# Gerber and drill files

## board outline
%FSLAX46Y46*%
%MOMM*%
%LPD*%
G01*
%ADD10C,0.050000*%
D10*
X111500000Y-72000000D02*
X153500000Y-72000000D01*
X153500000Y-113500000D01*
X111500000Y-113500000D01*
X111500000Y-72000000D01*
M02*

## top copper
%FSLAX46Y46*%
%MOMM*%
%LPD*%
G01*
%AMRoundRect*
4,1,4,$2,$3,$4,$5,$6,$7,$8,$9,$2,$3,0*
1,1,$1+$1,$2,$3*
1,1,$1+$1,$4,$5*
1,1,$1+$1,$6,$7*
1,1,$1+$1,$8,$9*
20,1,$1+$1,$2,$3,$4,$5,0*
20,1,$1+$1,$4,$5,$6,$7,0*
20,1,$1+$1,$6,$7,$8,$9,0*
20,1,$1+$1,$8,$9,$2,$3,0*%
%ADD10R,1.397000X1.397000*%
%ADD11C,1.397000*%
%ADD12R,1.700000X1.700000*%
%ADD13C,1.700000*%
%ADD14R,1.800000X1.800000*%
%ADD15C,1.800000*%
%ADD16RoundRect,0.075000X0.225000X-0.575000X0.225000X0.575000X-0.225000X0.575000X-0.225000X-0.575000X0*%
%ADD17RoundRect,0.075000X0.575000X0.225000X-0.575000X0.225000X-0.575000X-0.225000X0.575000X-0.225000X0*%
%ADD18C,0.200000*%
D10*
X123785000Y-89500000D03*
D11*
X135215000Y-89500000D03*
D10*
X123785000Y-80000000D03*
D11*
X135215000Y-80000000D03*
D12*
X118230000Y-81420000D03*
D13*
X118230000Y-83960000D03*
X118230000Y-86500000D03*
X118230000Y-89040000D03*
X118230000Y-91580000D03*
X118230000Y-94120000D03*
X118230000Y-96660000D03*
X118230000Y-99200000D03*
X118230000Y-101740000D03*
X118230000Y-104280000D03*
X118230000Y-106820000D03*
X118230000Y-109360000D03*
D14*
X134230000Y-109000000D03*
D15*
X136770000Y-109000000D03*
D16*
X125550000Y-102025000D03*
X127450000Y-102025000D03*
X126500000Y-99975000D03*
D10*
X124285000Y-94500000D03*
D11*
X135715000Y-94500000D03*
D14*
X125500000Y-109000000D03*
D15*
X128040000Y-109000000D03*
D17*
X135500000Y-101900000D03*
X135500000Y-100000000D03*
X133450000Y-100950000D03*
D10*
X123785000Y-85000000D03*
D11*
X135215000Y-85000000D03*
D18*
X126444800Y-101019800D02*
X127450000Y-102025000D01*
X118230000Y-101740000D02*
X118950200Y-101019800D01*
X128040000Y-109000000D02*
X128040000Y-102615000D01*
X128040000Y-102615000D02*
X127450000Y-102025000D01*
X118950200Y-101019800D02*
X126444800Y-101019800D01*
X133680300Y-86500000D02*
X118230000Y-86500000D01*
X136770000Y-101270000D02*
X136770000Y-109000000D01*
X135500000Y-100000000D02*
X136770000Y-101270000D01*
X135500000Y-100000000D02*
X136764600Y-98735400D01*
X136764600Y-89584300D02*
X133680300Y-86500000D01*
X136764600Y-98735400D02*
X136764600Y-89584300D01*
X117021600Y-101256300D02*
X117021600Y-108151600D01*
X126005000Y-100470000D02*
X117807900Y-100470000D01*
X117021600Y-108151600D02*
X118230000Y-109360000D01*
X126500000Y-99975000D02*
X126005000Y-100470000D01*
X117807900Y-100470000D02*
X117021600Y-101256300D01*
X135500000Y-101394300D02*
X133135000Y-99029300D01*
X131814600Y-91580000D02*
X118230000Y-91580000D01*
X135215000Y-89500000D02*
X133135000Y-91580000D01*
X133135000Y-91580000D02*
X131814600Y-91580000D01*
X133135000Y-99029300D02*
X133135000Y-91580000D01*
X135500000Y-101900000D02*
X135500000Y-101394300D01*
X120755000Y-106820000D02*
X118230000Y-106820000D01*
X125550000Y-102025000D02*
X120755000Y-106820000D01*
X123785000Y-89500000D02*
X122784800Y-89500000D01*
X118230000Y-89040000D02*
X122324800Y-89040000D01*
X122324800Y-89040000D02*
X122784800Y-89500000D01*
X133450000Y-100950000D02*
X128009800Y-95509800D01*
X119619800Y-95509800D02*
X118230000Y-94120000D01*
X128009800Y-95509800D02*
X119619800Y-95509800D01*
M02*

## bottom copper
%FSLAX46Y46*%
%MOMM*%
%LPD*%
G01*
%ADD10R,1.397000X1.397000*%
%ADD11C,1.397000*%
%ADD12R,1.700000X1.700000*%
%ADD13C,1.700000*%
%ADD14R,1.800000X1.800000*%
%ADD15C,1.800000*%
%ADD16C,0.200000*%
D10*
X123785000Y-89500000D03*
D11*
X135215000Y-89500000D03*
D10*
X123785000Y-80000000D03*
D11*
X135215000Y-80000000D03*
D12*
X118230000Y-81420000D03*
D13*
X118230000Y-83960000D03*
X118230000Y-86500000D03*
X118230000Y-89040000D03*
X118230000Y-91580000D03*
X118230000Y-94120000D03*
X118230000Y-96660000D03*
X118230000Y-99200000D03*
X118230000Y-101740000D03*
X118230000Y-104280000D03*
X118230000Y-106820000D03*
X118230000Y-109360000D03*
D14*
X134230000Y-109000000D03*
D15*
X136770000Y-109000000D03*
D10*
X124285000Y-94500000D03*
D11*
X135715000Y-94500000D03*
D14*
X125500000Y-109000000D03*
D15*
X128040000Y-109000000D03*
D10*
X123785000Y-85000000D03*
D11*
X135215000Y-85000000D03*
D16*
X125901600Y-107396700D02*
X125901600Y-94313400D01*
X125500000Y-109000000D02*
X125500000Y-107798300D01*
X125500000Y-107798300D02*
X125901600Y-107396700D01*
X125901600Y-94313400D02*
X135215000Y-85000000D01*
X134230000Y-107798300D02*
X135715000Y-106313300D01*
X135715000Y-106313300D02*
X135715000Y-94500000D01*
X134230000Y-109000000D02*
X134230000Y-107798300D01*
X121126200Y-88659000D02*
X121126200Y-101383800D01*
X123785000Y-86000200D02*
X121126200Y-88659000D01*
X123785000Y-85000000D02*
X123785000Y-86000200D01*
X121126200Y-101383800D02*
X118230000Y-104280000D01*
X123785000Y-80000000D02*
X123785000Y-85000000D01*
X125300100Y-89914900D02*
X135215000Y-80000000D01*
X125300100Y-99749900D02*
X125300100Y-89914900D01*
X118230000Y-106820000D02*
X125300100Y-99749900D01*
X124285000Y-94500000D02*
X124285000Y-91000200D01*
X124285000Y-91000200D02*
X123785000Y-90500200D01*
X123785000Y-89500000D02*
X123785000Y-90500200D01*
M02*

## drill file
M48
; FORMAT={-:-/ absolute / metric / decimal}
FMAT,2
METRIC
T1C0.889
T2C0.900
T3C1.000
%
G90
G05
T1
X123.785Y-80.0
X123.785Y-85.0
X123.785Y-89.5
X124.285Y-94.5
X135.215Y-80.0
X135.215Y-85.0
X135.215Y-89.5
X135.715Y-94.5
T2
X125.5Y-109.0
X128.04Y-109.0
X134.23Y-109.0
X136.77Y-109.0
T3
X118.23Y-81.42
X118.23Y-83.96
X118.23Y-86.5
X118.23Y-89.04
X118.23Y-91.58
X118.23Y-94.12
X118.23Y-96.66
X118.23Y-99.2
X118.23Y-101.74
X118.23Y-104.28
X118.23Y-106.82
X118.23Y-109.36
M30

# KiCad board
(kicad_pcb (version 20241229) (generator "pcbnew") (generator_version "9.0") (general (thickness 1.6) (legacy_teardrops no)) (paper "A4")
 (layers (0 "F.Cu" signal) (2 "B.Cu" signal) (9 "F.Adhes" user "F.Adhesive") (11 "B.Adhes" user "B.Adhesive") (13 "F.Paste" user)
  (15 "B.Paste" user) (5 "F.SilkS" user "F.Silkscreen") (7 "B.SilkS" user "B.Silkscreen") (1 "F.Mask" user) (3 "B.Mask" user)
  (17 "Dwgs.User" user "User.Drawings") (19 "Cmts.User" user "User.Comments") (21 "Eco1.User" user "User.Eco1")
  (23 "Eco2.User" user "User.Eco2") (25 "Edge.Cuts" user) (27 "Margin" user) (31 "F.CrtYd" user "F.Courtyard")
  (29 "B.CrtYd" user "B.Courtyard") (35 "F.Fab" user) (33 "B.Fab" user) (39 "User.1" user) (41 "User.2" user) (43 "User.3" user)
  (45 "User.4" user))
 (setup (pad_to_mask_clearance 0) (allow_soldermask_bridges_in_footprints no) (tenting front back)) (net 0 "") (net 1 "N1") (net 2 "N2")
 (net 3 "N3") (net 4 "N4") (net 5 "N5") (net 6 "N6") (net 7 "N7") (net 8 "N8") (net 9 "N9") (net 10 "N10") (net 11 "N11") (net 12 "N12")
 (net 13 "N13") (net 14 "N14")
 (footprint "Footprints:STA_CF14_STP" (layer "F.Cu") (at 123.785 89.5)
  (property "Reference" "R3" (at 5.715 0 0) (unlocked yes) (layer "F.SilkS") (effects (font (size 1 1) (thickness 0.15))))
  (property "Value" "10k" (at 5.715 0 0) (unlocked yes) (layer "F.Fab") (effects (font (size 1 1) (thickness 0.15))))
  (pad "1" thru_hole rect (at 0 0) (size 1.397 1.397) (drill 0.889) (layers "*.Cu" "*.Mask") (remove_unused_layers no) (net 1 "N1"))
  (pad "2" thru_hole circle (at 11.43 0) (size 1.397 1.397) (drill 0.889) (layers "*.Cu" "*.Mask") (remove_unused_layers no) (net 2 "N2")))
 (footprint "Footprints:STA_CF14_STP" (layer "F.Cu") (at 123.785 80)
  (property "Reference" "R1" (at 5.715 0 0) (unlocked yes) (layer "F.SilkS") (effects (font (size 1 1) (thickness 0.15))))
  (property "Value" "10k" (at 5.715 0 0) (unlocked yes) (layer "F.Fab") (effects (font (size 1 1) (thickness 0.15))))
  (pad "1" thru_hole rect (at 0 0) (size 1.397 1.397) (drill 0.889) (layers "*.Cu" "*.Mask") (remove_unused_layers no) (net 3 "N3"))
  (pad "2" thru_hole circle (at 11.43 0) (size 1.397 1.397) (drill 0.889) (layers "*.Cu" "*.Mask") (remove_unused_layers no) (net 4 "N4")))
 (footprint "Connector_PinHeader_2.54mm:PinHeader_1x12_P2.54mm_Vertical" (layer "F.Cu") (at 118.23 81.42)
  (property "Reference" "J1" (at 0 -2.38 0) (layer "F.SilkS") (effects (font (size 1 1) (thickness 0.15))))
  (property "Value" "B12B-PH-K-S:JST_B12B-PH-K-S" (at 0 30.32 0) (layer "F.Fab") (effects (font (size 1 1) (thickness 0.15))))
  (pad "1" thru_hole rect (at 0 0) (size 1.7 1.7) (drill 1) (layers "*.Cu" "*.Mask") (remove_unused_layers no) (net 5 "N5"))
  (pad "2" thru_hole circle (at 0 2.54) (size 1.7 1.7) (drill 1) (layers "*.Cu" "*.Mask") (remove_unused_layers no) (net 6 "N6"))
  (pad "3" thru_hole circle (at 0 5.08) (size 1.7 1.7) (drill 1) (layers "*.Cu" "*.Mask") (remove_unused_layers no) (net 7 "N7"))
  (pad "4" thru_hole circle (at 0 7.62) (size 1.7 1.7) (drill 1) (layers "*.Cu" "*.Mask") (remove_unused_layers no) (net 1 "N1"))
  (pad "5" thru_hole circle (at 0 10.16) (size 1.7 1.7) (drill 1) (layers "*.Cu" "*.Mask") (remove_unused_layers no) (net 2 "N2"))
  (pad "6" thru_hole circle (at 0 12.7) (size 1.7 1.7) (drill 1) (layers "*.Cu" "*.Mask") (remove_unused_layers no) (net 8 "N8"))
  (pad "7" thru_hole circle (at 0 15.24) (size 1.7 1.7) (drill 1) (layers "*.Cu" "*.Mask") (remove_unused_layers no) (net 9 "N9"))
  (pad "8" thru_hole circle (at 0 17.78) (size 1.7 1.7) (drill 1) (layers "*.Cu" "*.Mask") (remove_unused_layers no) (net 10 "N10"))
  (pad "9" thru_hole circle (at 0 20.32) (size 1.7 1.7) (drill 1) (layers "*.Cu" "*.Mask") (remove_unused_layers no) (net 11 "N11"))
  (pad "10" thru_hole circle (at 0 22.86) (size 1.7 1.7) (drill 1) (layers "*.Cu" "*.Mask") (remove_unused_layers no) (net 3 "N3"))
  (pad "11" thru_hole circle (at 0 25.4) (size 1.7 1.7) (drill 1) (layers "*.Cu" "*.Mask") (remove_unused_layers no) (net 4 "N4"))
  (pad "12" thru_hole circle (at 0 27.94) (size 1.7 1.7) (drill 1) (layers "*.Cu" "*.Mask") (remove_unused_layers no) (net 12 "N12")))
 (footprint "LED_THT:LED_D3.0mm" (layer "F.Cu") (at 134.23 109)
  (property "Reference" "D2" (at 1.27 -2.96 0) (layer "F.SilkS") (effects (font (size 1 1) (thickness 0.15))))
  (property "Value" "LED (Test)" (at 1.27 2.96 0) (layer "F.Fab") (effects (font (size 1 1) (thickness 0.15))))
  (pad "1" thru_hole rect (at 0 0) (size 1.8 1.8) (drill 0.9) (layers "*.Cu" "*.Mask") (remove_unused_layers no) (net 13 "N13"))
  (pad "2" thru_hole circle (at 2.54 0) (size 1.8 1.8) (drill 0.9) (layers "*.Cu" "*.Mask") (remove_unused_layers no) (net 7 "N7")))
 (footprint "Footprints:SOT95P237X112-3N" (layer "F.Cu") (at 126.5 101 90)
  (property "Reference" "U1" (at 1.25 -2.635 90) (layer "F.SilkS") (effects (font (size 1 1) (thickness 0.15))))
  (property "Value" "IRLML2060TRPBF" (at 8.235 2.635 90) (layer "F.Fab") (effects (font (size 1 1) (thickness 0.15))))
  (pad "1" smd roundrect (at -1.025 -0.95 90) (size 1.3 0.6) (layers "F.Cu" "F.Mask" "F.Paste") (roundrect_rratio 0.125) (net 4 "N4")
   (solder_mask_margin 0.102))
  (pad "2" smd roundrect (at -1.025 0.95 90) (size 1.3 0.6) (layers "F.Cu" "F.Mask" "F.Paste") (roundrect_rratio 0.125) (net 11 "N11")
   (solder_mask_margin 0.102))
  (pad "3" smd roundrect (at 1.025 0 90) (size 1.3 0.6) (layers "F.Cu" "F.Mask" "F.Paste") (roundrect_rratio 0.125) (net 12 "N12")
   (solder_mask_margin 0.102)))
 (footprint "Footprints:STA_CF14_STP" (layer "F.Cu") (at 124.285 94.5)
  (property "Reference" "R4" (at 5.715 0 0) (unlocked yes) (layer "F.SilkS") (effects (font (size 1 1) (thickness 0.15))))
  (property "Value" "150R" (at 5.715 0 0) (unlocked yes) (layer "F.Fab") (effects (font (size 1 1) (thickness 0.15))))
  (pad "1" thru_hole rect (at 0 0) (size 1.397 1.397) (drill 0.889) (layers "*.Cu" "*.Mask") (remove_unused_layers no) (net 1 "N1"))
  (pad "2" thru_hole circle (at 11.43 0) (size 1.397 1.397) (drill 0.889) (layers "*.Cu" "*.Mask") (remove_unused_layers no) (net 13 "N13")))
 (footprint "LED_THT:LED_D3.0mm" (layer "F.Cu") (at 125.5 109)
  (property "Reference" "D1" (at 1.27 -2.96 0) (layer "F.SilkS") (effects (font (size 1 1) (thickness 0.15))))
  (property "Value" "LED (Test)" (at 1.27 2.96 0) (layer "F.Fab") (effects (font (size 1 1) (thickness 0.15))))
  (pad "1" thru_hole rect (at 0 0) (size 1.8 1.8) (drill 0.9) (layers "*.Cu" "*.Mask") (remove_unused_layers no) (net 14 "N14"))
  (pad "2" thru_hole circle (at 2.54 0) (size 1.8 1.8) (drill 0.9) (layers "*.Cu" "*.Mask") (remove_unused_layers no) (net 11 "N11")))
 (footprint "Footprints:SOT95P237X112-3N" (layer "F.Cu") (at 134.475 100.95 180)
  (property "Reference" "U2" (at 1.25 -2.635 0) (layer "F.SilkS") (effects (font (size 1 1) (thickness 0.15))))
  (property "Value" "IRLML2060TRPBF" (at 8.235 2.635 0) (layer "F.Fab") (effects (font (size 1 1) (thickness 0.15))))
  (pad "1" smd roundrect (at -1.025 -0.95 180) (size 1.3 0.6) (layers "F.Cu" "F.Mask" "F.Paste") (roundrect_rratio 0.125) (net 2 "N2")
   (solder_mask_margin 0.102))
  (pad "2" smd roundrect (at -1.025 0.95 180) (size 1.3 0.6) (layers "F.Cu" "F.Mask" "F.Paste") (roundrect_rratio 0.125) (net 7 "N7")
   (solder_mask_margin 0.102))
  (pad "3" smd roundrect (at 1.025 0 180) (size 1.3 0.6) (layers "F.Cu" "F.Mask" "F.Paste") (roundrect_rratio 0.125) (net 8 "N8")
   (solder_mask_margin 0.102)))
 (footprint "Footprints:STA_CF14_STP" (layer "F.Cu") (at 123.785 85)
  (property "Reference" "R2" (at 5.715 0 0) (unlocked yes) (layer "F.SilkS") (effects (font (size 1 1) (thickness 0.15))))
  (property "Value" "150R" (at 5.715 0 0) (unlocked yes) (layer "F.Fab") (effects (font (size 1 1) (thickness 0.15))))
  (pad "1" thru_hole rect (at 0 0) (size 1.397 1.397) (drill 0.889) (layers "*.Cu" "*.Mask") (remove_unused_layers no) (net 3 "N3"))
  (pad "2" thru_hole circle (at 11.43 0) (size 1.397 1.397) (drill 0.889) (layers "*.Cu" "*.Mask") (remove_unused_layers no) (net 14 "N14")))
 (gr_rect (start 111.5 72) (end 153.5 113.5) (stroke (width 0.05) (type solid)) (fill no) (layer "Edge.Cuts"))
 (segment (start 125.9016 107.3967) (end 125.9016 94.3134) (width 0.2) (layer "B.Cu") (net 14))
 (segment (start 125.5 109) (end 125.5 107.7983) (width 0.2) (layer "B.Cu") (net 14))
 (segment (start 125.5 107.7983) (end 125.9016 107.3967) (width 0.2) (layer "B.Cu") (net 14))
 (segment (start 125.9016 94.3134) (end 135.215 85) (width 0.2) (layer "B.Cu") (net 14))
 (segment (start 126.4448 101.0198) (end 127.45 102.025) (width 0.2) (layer "F.Cu") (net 11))
 (segment (start 118.23 101.74) (end 118.9502 101.0198) (width 0.2) (layer "F.Cu") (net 11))
 (segment (start 128.04 109) (end 128.04 102.615) (width 0.2) (layer "F.Cu") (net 11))
 (segment (start 128.04 102.615) (end 127.45 102.025) (width 0.2) (layer "F.Cu") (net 11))
 (segment (start 118.9502 101.0198) (end 126.4448 101.0198) (width 0.2) (layer "F.Cu") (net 11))
 (segment (start 134.23 107.7983) (end 135.715 106.3133) (width 0.2) (layer "B.Cu") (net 13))
 (segment (start 135.715 106.3133) (end 135.715 94.5) (width 0.2) (layer "B.Cu") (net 13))
 (segment (start 134.23 109) (end 134.23 107.7983) (width 0.2) (layer "B.Cu") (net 13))
 (segment (start 133.6803 86.5) (end 118.23 86.5) (width 0.2) (layer "F.Cu") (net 7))
 (segment (start 136.77 101.27) (end 136.77 109) (width 0.2) (layer "F.Cu") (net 7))
 (segment (start 135.5 100) (end 136.77 101.27) (width 0.2) (layer "F.Cu") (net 7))
 (segment (start 135.5 100) (end 136.7646 98.7354) (width 0.2) (layer "F.Cu") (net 7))
 (segment (start 136.7646 89.5843) (end 133.6803 86.5) (width 0.2) (layer "F.Cu") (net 7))
 (segment (start 136.7646 98.7354) (end 136.7646 89.5843) (width 0.2) (layer "F.Cu") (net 7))
 (segment (start 117.0216 101.2563) (end 117.0216 108.1516) (width 0.2) (layer "F.Cu") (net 12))
 (segment (start 126.005 100.47) (end 117.8079 100.47) (width 0.2) (layer "F.Cu") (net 12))
 (segment (start 117.0216 108.1516) (end 118.23 109.36) (width 0.2) (layer "F.Cu") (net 12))
 (segment (start 126.5 99.975) (end 126.005 100.47) (width 0.2) (layer "F.Cu") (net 12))
 (segment (start 117.8079 100.47) (end 117.0216 101.2563) (width 0.2) (layer "F.Cu") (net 12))
 (segment (start 121.1262 88.659) (end 121.1262 101.3838) (width 0.2) (layer "B.Cu") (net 3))
 (segment (start 123.785 86.0002) (end 121.1262 88.659) (width 0.2) (layer "B.Cu") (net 3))
 (segment (start 123.785 85) (end 123.785 86.0002) (width 0.2) (layer "B.Cu") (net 3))
 (segment (start 121.1262 101.3838) (end 118.23 104.28) (width 0.2) (layer "B.Cu") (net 3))
 (segment (start 123.785 80) (end 123.785 85) (width 0.2) (layer "B.Cu") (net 3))
 (segment (start 135.5 101.3943) (end 133.135 99.0293) (width 0.2) (layer "F.Cu") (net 2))
 (segment (start 131.8146 91.58) (end 118.23 91.58) (width 0.2) (layer "F.Cu") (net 2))
 (segment (start 135.215 89.5) (end 133.135 91.58) (width 0.2) (layer "F.Cu") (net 2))
 (segment (start 133.135 91.58) (end 131.8146 91.58) (width 0.2) (layer "F.Cu") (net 2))
 (segment (start 133.135 99.0293) (end 133.135 91.58) (width 0.2) (layer "F.Cu") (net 2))
 (segment (start 135.5 101.9) (end 135.5 101.3943) (width 0.2) (layer "F.Cu") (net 2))
 (segment (start 120.755 106.82) (end 118.23 106.82) (width 0.2) (layer "F.Cu") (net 4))
 (segment (start 125.55 102.025) (end 120.755 106.82) (width 0.2) (layer "F.Cu") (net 4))
 (segment (start 125.3001 89.9149) (end 135.215 80) (width 0.2) (layer "B.Cu") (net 4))
 (segment (start 125.3001 99.7499) (end 125.3001 89.9149) (width 0.2) (layer "B.Cu") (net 4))
 (segment (start 118.23 106.82) (end 125.3001 99.7499) (width 0.2) (layer "B.Cu") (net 4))
 (segment (start 123.785 89.5) (end 122.7848 89.5) (width 0.2) (layer "F.Cu") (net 1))
 (segment (start 118.23 89.04) (end 122.3248 89.04) (width 0.2) (layer "F.Cu") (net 1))
 (segment (start 122.3248 89.04) (end 122.7848 89.5) (width 0.2) (layer "F.Cu") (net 1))
 (segment (start 124.285 94.5) (end 124.285 91.0002) (width 0.2) (layer "B.Cu") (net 1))
 (segment (start 124.285 91.0002) (end 123.785 90.5002) (width 0.2) (layer "B.Cu") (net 1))
 (segment (start 123.785 89.5) (end 123.785 90.5002) (width 0.2) (layer "B.Cu") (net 1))
 (segment (start 133.45 100.95) (end 128.0098 95.5098) (width 0.2) (layer "F.Cu") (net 8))
 (segment (start 119.6198 95.5098) (end 118.23 94.12) (width 0.2) (layer "F.Cu") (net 8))
 (segment (start 128.0098 95.5098) (end 119.6198 95.5098) (width 0.2) (layer "F.Cu") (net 8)))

